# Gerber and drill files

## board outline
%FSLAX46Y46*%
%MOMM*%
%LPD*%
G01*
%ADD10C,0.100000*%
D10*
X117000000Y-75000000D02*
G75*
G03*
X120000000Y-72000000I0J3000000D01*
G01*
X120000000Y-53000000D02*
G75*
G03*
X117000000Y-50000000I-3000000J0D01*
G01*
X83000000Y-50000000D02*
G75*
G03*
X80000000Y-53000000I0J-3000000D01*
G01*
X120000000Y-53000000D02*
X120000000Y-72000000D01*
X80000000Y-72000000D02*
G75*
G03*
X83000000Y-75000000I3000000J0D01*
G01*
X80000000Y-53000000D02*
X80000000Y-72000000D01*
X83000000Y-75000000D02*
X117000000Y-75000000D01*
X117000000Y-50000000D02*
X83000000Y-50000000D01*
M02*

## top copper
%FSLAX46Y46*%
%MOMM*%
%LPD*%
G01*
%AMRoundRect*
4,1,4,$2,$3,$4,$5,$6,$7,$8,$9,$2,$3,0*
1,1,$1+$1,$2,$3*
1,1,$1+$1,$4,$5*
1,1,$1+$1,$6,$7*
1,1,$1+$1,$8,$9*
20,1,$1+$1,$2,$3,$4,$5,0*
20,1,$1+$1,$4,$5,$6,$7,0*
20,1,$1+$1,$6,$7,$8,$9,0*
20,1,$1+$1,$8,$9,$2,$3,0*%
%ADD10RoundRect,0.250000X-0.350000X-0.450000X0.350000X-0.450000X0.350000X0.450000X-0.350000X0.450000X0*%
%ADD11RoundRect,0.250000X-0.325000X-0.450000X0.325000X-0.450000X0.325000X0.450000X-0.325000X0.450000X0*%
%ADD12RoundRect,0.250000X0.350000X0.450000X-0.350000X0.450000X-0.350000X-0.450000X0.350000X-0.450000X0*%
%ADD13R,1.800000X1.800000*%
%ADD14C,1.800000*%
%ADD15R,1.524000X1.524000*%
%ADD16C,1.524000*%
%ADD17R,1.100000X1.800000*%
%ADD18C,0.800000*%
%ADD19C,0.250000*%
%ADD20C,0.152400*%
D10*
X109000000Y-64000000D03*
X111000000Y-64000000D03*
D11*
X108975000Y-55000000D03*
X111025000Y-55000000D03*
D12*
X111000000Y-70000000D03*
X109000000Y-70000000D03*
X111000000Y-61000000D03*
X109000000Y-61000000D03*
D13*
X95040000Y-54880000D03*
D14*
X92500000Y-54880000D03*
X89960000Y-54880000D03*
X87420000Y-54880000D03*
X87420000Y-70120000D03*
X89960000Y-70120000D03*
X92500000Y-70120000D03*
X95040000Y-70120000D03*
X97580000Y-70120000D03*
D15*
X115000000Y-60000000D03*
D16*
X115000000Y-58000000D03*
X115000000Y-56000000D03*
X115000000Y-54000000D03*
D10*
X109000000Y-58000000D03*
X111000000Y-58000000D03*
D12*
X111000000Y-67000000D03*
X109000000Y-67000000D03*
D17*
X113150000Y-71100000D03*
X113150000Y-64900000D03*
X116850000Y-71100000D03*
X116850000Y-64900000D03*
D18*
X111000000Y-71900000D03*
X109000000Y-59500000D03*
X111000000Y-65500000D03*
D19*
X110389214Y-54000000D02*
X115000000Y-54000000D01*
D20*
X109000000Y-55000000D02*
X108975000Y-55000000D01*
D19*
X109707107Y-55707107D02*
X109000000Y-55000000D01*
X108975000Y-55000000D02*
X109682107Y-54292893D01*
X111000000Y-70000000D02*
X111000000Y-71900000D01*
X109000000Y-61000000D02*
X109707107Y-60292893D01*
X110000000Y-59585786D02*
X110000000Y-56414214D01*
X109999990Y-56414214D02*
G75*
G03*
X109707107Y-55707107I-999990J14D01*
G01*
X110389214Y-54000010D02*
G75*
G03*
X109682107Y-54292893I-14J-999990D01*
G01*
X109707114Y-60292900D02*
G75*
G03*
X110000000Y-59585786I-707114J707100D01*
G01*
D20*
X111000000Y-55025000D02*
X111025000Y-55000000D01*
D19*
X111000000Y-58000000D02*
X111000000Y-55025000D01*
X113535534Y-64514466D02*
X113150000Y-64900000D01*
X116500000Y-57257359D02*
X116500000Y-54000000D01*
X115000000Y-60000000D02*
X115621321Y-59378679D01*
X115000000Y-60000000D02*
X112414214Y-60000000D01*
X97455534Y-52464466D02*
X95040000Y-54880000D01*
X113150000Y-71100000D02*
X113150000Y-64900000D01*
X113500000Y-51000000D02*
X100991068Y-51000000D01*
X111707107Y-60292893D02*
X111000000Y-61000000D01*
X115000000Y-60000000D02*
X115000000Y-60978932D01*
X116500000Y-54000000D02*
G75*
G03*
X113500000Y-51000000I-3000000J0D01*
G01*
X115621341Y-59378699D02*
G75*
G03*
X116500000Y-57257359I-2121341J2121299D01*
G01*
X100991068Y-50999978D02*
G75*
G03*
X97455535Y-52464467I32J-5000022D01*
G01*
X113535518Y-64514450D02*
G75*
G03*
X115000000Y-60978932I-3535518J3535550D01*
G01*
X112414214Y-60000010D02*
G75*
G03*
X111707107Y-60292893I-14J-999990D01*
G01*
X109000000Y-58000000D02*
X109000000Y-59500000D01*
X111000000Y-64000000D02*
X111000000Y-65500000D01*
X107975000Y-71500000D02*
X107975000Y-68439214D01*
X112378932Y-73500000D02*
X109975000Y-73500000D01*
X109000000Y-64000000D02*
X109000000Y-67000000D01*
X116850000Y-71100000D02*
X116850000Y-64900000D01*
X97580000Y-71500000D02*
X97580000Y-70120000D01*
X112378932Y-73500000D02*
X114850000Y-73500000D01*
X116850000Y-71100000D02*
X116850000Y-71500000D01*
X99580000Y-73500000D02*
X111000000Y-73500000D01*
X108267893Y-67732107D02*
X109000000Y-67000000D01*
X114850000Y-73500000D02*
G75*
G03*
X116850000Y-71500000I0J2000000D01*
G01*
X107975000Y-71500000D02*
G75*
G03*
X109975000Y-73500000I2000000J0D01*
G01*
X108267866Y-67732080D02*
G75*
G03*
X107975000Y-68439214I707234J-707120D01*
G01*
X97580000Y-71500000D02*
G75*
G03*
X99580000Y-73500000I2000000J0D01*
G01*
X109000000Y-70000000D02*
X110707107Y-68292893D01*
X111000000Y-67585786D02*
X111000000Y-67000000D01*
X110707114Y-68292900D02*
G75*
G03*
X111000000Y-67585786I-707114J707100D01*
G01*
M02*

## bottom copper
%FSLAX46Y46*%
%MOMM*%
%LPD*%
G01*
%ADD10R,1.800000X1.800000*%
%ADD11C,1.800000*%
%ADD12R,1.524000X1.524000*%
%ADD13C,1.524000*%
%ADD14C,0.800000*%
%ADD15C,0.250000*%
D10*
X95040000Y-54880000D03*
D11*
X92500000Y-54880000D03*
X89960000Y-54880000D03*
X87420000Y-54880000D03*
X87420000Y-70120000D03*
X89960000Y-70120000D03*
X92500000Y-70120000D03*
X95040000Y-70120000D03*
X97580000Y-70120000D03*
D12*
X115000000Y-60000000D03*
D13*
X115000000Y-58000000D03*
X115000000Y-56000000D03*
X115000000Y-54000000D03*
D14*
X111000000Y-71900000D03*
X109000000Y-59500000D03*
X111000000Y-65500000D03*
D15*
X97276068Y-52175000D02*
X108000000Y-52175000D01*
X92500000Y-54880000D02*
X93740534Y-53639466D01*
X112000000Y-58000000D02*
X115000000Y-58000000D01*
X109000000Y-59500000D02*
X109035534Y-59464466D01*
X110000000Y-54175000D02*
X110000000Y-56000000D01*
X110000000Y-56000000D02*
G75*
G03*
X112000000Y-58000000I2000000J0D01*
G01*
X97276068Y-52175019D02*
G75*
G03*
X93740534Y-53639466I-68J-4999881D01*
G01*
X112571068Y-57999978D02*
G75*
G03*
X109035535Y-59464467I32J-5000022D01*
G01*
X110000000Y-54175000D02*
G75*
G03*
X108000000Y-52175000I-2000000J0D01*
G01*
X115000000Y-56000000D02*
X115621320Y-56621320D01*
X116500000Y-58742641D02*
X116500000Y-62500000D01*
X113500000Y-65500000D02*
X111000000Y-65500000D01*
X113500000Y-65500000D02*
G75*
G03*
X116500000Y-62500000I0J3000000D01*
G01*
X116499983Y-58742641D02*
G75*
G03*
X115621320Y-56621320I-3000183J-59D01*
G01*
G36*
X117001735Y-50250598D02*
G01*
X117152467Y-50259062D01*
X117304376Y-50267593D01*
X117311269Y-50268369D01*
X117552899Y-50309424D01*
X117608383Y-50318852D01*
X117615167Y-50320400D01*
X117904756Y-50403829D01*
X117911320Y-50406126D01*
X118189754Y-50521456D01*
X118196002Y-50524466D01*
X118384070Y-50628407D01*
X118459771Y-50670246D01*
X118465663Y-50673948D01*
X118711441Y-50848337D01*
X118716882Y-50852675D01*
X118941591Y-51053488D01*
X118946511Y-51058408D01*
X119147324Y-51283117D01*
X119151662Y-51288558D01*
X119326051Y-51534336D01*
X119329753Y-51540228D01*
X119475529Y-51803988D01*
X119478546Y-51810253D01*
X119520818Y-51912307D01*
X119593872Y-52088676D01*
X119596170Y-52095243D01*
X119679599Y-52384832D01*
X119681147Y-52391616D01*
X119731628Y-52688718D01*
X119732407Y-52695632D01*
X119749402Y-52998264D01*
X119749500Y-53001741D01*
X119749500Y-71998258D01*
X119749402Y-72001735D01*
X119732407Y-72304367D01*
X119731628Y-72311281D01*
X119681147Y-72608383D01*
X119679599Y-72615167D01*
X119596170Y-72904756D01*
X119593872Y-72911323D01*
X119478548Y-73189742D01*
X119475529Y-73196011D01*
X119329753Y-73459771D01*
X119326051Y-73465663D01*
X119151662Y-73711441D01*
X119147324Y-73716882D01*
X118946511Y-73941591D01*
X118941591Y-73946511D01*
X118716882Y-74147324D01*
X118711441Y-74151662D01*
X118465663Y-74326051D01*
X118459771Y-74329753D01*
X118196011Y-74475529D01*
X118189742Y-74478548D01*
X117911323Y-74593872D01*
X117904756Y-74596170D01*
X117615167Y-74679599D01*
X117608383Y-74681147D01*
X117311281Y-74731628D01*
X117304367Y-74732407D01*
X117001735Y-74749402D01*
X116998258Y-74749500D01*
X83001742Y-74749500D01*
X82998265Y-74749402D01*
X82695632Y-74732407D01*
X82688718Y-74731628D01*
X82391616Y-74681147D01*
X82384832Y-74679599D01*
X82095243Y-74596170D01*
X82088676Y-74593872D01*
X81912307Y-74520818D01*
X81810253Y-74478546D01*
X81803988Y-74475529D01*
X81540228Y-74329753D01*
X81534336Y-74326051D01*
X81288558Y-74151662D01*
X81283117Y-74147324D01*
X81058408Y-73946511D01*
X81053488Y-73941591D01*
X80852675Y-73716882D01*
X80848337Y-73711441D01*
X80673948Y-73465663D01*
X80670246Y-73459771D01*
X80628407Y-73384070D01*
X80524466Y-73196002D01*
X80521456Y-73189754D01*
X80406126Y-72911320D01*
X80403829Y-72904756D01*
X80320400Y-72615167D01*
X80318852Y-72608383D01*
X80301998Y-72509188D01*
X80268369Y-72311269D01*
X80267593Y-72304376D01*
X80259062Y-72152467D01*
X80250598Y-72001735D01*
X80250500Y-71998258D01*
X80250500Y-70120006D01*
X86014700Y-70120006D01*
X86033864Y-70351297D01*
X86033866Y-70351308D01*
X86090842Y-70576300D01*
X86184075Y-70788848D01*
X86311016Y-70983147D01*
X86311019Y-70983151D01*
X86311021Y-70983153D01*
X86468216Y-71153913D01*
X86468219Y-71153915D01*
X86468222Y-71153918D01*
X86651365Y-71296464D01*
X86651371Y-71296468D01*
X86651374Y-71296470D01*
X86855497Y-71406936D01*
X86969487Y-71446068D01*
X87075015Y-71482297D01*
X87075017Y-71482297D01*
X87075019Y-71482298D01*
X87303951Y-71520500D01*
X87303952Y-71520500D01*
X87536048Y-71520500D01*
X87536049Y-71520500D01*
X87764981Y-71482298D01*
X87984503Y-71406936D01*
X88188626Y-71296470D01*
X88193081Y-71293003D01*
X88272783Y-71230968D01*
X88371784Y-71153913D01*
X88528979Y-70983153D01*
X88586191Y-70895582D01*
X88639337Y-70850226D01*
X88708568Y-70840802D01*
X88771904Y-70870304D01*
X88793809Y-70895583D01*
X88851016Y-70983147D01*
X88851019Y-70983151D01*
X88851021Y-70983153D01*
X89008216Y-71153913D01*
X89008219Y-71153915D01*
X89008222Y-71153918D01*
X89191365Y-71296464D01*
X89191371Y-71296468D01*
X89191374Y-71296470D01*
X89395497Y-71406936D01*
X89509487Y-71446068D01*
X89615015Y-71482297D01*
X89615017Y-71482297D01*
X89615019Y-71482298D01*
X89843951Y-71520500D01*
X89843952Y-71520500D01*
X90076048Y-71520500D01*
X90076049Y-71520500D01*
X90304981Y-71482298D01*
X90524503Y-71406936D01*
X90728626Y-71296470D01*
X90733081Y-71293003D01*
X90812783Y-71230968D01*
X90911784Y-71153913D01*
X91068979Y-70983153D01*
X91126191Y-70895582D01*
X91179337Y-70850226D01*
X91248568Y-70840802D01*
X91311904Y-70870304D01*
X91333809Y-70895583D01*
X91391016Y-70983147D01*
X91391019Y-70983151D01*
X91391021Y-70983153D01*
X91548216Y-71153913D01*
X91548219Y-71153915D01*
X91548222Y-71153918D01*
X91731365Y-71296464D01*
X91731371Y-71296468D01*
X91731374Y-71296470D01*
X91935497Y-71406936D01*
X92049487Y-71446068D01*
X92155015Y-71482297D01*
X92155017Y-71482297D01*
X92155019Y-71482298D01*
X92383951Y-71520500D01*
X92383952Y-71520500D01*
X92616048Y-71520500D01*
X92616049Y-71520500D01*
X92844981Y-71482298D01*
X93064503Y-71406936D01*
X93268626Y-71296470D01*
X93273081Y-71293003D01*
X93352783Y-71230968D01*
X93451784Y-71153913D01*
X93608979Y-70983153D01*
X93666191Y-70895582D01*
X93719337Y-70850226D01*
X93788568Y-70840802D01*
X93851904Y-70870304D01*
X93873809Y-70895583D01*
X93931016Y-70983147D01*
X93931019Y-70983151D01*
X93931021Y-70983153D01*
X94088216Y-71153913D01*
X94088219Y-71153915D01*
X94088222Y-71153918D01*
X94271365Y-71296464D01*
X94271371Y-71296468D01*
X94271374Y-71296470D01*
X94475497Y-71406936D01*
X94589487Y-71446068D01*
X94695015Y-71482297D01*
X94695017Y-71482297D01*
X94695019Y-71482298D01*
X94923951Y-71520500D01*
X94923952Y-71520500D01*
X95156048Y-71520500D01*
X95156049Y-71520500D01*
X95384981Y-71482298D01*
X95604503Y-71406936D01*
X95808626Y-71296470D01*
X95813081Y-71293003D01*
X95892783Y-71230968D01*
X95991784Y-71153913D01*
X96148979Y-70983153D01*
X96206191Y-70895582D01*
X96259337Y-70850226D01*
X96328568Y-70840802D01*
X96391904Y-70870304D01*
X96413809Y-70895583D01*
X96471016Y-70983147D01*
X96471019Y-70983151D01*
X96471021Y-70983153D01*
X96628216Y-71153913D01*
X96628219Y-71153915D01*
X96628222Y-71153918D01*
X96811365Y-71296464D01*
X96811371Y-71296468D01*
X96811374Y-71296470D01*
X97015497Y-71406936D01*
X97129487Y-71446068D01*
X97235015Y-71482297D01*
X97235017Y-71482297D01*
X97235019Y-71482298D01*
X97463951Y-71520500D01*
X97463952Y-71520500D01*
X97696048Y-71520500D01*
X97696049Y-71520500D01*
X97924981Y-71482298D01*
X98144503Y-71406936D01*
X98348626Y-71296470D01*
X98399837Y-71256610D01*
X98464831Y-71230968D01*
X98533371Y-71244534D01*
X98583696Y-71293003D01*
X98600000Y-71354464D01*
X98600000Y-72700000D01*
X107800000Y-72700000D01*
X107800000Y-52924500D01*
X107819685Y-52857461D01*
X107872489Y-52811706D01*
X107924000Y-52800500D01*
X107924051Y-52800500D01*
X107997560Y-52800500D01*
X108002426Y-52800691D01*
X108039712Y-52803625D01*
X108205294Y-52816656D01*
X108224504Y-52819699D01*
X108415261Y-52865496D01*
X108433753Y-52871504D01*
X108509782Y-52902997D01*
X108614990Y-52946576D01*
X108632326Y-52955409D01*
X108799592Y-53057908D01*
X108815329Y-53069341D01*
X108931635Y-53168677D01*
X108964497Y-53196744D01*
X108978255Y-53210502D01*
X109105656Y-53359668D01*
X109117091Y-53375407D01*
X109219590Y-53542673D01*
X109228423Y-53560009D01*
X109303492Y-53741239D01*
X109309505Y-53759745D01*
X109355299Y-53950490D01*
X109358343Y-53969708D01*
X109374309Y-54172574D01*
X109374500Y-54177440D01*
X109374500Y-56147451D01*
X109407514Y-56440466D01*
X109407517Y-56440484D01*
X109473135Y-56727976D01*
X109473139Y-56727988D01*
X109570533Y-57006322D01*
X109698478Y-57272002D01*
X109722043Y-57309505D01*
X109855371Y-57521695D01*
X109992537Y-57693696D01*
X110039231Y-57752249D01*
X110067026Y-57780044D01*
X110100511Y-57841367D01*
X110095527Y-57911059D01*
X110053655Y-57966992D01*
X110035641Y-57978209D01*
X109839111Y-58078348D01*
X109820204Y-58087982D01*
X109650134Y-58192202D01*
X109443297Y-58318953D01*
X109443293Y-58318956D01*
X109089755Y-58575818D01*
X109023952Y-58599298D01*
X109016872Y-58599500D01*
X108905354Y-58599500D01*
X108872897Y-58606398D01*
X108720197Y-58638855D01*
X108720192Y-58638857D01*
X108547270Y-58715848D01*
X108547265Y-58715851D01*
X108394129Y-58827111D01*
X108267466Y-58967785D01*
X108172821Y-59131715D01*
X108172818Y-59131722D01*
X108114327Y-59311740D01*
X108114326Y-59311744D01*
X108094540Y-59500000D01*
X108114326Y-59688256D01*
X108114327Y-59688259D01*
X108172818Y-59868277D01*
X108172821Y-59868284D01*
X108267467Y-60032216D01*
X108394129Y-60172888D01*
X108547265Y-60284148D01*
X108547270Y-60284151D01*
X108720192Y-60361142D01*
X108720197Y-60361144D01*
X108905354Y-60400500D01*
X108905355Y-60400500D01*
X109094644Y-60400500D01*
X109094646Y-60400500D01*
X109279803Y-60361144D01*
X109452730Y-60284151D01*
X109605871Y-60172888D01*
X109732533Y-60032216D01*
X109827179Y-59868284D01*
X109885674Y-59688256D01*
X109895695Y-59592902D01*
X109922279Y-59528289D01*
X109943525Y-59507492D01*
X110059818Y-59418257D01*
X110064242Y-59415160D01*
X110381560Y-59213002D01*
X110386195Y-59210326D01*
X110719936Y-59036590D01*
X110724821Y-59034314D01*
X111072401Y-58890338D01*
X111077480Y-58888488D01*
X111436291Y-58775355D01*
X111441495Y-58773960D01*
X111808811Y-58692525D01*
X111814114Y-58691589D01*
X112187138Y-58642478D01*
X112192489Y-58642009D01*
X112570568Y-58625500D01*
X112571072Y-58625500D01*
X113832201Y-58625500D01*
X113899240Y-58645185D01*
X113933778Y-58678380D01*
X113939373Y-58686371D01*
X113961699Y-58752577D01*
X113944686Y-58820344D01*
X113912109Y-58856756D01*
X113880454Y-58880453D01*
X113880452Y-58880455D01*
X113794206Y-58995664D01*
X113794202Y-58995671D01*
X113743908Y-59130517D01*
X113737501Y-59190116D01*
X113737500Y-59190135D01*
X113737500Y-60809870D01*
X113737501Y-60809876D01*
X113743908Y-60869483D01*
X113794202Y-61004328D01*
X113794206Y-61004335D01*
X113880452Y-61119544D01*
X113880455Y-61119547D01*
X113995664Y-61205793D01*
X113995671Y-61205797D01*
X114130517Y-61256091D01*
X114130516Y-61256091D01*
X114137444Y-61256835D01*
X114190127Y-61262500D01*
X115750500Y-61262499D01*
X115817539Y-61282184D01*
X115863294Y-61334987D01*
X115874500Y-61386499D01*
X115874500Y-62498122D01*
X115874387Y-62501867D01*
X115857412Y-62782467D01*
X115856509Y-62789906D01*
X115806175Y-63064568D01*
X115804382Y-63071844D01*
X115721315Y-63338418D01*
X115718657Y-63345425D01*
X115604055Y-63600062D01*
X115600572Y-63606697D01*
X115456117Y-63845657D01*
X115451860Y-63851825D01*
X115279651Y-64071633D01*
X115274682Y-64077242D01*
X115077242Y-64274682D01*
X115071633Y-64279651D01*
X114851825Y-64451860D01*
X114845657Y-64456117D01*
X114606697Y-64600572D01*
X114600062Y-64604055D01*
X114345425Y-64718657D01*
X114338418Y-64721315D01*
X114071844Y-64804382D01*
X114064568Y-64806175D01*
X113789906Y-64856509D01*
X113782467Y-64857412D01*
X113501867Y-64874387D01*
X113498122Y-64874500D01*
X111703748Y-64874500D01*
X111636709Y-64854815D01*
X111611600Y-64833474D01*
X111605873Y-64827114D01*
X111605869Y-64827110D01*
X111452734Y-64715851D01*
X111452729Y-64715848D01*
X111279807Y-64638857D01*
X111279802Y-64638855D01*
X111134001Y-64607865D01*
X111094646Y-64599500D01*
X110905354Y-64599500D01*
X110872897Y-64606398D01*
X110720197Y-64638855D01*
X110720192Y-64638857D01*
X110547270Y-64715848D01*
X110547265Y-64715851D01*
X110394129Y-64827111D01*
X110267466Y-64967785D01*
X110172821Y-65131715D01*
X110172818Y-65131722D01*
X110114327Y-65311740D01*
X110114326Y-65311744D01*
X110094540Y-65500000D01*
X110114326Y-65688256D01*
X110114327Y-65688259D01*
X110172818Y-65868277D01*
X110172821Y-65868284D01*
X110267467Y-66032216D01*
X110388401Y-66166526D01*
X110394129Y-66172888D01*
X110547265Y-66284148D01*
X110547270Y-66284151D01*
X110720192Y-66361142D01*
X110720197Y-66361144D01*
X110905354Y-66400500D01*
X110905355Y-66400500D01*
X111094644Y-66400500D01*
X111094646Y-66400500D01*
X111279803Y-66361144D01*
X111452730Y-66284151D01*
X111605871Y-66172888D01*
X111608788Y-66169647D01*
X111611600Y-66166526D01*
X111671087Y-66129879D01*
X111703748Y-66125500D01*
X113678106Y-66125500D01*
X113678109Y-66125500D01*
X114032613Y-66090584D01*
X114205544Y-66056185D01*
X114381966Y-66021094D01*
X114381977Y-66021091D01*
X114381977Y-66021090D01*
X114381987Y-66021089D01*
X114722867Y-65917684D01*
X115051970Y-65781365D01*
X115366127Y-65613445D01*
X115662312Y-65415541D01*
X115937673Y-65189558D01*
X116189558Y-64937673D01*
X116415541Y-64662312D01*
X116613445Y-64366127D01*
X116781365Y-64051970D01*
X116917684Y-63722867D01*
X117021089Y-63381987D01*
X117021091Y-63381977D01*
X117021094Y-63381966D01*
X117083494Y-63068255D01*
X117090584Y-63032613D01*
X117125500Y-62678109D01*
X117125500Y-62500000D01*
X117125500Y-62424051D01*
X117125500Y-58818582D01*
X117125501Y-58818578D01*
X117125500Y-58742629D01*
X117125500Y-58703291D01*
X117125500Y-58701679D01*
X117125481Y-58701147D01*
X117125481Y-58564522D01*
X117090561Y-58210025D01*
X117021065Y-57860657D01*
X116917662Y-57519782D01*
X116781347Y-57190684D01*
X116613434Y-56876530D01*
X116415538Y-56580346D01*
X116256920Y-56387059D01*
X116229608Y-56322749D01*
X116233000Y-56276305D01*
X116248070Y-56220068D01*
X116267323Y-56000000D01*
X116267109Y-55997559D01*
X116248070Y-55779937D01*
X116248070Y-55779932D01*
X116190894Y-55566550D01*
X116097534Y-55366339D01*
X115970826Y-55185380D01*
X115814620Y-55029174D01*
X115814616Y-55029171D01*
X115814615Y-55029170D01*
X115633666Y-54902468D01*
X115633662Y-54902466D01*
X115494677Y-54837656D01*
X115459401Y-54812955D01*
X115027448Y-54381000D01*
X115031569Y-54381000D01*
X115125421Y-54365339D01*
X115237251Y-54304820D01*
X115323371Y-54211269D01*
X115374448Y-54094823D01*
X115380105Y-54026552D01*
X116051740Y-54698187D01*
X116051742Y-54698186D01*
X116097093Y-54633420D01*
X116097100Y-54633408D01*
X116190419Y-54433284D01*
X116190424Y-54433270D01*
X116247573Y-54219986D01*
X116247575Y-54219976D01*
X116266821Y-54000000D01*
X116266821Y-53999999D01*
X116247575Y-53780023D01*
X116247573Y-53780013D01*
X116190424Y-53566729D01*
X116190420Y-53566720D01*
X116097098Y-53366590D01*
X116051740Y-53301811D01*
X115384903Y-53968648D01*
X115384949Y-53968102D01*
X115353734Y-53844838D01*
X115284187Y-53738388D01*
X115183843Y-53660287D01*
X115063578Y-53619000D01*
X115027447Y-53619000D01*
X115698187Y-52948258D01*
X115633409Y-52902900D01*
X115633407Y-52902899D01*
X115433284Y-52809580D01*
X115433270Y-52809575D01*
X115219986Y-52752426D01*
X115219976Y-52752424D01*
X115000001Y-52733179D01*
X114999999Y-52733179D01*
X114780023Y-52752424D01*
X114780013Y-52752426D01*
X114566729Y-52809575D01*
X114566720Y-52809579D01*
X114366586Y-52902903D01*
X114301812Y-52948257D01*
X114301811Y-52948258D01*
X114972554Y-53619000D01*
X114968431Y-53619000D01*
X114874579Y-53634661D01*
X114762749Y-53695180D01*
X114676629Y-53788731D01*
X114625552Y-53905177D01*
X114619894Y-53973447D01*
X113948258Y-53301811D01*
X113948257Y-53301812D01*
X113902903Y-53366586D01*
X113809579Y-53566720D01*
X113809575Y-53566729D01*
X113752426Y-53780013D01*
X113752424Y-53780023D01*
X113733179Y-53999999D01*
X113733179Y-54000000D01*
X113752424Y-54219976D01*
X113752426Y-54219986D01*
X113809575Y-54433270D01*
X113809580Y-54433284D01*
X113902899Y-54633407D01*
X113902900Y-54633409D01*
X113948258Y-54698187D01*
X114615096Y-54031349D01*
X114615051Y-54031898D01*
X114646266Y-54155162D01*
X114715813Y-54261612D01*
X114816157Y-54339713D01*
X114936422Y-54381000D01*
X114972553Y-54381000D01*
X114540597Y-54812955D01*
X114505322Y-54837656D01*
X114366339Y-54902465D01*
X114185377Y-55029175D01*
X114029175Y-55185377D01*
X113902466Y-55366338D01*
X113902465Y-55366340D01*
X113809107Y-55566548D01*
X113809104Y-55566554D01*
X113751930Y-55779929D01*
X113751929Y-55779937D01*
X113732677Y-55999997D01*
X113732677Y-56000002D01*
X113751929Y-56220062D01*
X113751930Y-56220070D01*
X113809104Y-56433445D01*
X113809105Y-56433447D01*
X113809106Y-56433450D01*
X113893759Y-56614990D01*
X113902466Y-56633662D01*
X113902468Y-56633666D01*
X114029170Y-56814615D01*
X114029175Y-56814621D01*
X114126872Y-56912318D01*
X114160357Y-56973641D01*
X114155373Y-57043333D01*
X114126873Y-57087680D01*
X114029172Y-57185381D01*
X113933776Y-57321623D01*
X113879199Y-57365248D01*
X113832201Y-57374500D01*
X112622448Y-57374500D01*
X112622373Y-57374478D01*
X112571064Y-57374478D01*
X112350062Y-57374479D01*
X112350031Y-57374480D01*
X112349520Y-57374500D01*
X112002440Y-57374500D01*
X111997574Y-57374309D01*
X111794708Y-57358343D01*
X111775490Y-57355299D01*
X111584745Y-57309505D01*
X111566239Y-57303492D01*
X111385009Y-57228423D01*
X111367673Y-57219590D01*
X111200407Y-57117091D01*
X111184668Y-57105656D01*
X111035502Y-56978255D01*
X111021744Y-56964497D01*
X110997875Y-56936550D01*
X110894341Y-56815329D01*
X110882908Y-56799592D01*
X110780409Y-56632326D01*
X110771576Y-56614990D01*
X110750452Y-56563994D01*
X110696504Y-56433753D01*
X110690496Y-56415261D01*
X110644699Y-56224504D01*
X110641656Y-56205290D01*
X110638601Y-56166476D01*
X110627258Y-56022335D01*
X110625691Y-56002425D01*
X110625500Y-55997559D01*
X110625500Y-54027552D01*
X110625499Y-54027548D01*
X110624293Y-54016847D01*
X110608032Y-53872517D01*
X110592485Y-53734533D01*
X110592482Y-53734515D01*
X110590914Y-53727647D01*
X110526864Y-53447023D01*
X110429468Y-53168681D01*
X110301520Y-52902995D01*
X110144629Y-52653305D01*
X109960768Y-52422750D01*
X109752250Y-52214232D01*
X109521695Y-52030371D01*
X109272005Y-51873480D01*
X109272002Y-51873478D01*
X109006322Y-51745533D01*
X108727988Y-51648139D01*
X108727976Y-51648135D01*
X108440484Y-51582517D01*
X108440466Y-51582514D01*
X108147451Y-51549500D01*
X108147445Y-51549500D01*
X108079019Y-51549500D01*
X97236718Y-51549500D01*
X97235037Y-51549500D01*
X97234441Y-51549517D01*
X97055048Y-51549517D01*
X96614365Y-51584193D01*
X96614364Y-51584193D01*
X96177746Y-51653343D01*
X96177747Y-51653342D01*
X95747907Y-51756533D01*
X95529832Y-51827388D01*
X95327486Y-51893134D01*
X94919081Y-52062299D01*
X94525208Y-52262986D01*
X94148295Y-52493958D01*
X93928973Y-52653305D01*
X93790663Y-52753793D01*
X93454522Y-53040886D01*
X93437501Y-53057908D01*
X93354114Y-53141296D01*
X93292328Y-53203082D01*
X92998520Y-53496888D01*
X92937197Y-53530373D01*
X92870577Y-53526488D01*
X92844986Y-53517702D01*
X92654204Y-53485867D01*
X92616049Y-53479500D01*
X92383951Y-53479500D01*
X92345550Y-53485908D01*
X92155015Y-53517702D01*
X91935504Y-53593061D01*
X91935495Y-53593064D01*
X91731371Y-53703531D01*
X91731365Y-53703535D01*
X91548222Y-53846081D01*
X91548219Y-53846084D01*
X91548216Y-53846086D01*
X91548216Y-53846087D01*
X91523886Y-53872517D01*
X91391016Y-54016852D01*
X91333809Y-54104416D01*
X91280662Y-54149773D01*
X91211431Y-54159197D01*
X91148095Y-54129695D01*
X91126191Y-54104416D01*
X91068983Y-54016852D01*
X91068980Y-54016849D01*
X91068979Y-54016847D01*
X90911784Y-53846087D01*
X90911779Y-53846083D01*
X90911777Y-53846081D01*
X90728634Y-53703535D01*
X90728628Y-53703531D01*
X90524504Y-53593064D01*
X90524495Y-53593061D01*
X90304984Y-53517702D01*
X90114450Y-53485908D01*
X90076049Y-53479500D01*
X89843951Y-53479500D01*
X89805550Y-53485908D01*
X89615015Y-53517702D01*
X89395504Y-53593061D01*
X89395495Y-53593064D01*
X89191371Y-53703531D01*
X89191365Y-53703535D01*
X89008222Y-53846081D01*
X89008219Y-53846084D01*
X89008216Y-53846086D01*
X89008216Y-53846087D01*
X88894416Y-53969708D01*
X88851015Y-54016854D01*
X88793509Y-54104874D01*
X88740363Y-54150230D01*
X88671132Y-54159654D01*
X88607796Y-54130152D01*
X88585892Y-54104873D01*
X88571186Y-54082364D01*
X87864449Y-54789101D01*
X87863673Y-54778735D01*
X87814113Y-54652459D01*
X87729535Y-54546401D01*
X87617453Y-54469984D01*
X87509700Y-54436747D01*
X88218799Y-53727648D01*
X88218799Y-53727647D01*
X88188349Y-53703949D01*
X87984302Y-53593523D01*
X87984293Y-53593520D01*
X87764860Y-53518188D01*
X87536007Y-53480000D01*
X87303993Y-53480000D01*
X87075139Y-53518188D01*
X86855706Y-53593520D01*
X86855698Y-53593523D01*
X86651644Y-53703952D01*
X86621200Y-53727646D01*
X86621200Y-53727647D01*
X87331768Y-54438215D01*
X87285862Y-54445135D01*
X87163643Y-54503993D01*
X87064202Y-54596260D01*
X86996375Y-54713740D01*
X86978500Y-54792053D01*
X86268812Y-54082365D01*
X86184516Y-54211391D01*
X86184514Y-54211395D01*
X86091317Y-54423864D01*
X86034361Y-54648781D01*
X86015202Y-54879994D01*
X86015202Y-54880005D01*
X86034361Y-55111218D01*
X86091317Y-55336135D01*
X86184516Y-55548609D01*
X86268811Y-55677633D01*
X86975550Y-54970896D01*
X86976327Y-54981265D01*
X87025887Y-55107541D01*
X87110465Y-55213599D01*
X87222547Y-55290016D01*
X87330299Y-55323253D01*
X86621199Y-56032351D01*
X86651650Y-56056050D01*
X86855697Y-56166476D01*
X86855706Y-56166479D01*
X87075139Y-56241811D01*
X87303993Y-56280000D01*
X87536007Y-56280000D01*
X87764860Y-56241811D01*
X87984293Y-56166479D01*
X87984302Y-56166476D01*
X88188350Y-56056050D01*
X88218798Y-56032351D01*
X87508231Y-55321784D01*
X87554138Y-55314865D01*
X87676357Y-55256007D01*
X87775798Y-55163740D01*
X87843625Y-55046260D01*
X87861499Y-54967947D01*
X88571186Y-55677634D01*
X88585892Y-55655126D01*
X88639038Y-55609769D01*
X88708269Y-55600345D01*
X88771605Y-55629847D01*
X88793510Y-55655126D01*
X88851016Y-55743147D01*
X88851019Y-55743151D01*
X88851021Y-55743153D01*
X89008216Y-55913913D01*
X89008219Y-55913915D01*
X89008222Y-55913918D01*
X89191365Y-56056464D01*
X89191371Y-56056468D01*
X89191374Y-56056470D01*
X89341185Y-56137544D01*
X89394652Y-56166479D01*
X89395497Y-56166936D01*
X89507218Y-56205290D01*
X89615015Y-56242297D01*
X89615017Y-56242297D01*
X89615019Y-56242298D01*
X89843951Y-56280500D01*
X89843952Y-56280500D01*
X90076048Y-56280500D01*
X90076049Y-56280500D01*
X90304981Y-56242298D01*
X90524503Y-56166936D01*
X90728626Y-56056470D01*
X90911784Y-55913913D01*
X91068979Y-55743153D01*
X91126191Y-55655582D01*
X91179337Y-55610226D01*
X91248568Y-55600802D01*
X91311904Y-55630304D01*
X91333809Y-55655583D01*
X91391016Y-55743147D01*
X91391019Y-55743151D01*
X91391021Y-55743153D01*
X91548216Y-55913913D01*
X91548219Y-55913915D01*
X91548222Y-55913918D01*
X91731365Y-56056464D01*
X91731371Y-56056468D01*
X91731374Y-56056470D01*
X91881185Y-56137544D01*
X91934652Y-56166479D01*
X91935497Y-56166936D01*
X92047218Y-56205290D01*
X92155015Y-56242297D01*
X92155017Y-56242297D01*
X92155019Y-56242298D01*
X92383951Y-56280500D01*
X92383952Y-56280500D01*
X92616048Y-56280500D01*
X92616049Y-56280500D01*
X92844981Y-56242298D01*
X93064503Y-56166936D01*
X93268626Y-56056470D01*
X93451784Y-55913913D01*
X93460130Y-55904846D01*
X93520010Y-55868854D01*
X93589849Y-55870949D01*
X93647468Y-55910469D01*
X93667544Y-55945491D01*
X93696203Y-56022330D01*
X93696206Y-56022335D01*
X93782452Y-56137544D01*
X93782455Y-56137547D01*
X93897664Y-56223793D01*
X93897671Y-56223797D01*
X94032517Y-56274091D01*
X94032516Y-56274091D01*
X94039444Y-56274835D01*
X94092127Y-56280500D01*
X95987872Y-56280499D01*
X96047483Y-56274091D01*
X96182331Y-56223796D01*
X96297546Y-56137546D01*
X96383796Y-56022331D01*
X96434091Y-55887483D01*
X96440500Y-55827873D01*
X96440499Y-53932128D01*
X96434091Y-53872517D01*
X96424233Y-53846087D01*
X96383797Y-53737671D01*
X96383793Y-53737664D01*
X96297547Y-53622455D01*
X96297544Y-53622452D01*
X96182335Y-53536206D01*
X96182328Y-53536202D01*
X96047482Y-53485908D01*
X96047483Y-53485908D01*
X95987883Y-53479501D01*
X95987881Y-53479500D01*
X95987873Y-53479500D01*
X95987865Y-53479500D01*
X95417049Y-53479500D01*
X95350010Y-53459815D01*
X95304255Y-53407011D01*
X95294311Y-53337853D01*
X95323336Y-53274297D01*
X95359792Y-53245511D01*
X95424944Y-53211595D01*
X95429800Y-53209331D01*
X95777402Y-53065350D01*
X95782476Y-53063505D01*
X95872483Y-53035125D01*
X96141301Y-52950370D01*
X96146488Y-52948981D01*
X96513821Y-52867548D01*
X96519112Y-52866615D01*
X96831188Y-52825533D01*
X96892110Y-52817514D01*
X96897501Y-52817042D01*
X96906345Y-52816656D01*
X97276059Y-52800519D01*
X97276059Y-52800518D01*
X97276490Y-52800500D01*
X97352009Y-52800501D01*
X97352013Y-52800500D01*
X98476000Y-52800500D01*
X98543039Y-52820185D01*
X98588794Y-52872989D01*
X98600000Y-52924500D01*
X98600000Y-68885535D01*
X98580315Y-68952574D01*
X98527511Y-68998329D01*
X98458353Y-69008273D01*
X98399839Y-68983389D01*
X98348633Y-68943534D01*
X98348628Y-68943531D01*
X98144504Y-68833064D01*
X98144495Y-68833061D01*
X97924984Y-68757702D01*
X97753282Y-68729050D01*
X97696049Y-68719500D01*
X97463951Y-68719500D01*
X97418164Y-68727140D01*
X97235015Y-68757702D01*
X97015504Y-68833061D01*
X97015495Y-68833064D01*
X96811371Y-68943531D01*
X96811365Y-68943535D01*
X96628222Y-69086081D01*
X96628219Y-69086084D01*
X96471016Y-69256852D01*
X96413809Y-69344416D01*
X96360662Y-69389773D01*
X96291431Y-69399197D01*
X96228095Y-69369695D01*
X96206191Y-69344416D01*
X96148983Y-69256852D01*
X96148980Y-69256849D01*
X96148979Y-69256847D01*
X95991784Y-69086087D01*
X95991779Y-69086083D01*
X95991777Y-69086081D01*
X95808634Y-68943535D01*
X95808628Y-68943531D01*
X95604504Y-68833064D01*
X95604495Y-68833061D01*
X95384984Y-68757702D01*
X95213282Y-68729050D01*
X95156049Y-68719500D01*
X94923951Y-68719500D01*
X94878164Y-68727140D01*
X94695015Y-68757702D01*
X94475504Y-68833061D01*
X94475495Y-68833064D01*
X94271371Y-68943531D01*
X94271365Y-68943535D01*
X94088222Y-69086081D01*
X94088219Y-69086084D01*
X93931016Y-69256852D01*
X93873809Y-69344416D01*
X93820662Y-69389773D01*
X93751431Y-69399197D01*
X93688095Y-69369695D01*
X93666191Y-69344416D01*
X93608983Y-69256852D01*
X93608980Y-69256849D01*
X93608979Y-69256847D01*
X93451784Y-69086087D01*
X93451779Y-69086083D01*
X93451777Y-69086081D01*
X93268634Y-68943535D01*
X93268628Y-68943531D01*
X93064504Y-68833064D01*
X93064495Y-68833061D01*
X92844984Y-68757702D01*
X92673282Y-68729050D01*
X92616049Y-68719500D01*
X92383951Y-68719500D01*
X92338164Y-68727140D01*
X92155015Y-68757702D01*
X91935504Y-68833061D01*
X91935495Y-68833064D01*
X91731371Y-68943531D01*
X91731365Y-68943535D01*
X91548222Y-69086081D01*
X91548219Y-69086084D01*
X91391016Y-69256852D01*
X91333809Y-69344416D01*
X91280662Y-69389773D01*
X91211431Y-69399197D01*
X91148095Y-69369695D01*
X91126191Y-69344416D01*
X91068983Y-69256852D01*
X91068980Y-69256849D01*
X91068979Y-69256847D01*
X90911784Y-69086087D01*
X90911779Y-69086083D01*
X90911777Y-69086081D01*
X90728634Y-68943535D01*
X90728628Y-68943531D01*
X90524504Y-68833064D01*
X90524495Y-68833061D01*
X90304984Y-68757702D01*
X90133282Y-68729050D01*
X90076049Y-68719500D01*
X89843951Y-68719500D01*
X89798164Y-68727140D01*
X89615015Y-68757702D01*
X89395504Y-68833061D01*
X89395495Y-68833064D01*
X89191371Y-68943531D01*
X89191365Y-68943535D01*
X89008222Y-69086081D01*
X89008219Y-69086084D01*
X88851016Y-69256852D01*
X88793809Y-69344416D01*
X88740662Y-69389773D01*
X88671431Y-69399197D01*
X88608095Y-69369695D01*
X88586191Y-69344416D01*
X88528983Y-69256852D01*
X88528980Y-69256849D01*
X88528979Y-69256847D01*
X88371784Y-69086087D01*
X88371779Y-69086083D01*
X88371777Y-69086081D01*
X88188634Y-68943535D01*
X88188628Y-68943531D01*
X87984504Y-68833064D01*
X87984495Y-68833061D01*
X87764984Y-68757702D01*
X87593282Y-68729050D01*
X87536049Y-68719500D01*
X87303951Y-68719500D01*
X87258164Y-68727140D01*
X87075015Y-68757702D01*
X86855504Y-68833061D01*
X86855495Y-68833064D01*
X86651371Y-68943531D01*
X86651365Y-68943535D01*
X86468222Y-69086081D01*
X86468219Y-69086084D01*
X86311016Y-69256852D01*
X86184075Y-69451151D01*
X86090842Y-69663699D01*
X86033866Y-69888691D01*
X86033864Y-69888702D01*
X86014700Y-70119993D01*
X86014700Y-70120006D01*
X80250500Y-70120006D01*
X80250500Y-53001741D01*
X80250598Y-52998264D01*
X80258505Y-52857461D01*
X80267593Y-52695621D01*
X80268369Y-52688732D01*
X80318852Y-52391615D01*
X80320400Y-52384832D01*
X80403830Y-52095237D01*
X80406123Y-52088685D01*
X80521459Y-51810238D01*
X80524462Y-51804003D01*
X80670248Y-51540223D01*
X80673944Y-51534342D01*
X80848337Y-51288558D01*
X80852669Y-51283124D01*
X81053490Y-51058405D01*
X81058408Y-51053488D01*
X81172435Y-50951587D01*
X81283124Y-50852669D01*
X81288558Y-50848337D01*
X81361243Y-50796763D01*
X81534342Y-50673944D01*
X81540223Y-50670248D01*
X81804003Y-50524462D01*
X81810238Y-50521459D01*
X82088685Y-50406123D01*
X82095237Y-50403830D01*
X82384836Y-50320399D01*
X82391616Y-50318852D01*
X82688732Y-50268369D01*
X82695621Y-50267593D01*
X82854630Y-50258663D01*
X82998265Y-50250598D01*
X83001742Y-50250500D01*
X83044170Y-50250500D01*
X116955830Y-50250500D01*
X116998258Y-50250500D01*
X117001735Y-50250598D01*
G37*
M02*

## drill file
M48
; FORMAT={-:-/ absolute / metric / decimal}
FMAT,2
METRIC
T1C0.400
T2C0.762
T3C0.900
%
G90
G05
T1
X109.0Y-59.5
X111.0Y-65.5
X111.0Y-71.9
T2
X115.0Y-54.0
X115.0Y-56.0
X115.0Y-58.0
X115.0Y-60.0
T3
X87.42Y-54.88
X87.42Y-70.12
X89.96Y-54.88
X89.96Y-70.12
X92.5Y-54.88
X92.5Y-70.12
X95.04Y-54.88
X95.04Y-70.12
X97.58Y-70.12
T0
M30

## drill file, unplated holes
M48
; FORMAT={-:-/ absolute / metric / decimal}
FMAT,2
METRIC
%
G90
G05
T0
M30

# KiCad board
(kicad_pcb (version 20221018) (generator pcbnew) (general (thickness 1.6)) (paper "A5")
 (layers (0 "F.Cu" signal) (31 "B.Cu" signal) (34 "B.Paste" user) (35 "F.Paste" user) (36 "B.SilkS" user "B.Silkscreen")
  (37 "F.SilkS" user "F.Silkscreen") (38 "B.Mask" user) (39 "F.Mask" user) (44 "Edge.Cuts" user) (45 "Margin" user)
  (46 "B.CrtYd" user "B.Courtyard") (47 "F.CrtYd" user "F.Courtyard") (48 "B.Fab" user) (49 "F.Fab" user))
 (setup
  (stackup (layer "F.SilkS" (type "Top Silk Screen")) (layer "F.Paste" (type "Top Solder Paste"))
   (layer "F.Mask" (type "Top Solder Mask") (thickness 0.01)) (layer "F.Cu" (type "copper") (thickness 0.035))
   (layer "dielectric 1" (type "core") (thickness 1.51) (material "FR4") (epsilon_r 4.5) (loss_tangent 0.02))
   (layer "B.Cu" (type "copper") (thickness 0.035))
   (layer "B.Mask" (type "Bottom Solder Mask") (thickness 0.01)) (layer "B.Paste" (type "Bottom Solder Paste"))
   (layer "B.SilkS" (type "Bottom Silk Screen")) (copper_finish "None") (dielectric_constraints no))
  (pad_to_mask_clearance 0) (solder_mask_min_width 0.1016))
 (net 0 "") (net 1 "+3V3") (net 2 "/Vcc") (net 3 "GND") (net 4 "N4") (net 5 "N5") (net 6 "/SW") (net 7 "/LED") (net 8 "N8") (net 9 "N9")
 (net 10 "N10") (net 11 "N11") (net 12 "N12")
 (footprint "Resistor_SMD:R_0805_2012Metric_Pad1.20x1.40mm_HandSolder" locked (layer "F.Cu") (at 110 64)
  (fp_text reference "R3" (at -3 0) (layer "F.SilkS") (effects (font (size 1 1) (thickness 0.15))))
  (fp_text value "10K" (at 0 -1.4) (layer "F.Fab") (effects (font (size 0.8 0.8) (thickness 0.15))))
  (pad "1" smd roundrect locked (at -1 0) (size 1.2 1.4) (layers "F.Cu" "F.Paste" "F.Mask") (roundrect_rratio 0.2083333333) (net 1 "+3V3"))
  (pad "2" smd roundrect locked (at 1 0) (size 1.2 1.4) (layers "F.Cu" "F.Paste" "F.Mask") (roundrect_rratio 0.2083333333) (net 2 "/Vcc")))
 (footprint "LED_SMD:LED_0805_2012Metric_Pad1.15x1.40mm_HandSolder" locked (layer "F.Cu") (at 110 55)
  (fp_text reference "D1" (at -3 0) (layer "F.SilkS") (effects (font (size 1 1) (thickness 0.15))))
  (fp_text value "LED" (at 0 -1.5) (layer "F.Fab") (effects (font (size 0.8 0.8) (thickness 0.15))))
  (pad "1" smd roundrect locked (at -1.025 0) (size 1.15 1.4) (layers "F.Cu" "F.Paste" "F.Mask") (roundrect_rratio 0.2173913043)
   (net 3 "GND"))
  (pad "2" smd roundrect locked (at 1.025 0) (size 1.15 1.4) (layers "F.Cu" "F.Paste" "F.Mask") (roundrect_rratio 0.2173913043) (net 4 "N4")))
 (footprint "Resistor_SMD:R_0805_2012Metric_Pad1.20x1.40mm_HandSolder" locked (layer "F.Cu") (at 110 70 180)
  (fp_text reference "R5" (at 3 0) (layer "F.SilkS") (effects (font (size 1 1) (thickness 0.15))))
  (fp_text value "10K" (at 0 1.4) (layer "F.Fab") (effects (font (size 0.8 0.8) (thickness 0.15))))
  (pad "1" smd roundrect locked (at -1 0 180) (size 1.2 1.4) (layers "F.Cu" "F.Paste" "F.Mask") (roundrect_rratio 0.2083333333)
   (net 3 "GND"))
  (pad "2" smd roundrect locked (at 1 0 180) (size 1.2 1.4) (layers "F.Cu" "F.Paste" "F.Mask") (roundrect_rratio 0.2083333333) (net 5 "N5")))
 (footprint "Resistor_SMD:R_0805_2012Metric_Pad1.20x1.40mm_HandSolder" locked (layer "F.Cu") (at 110 61 180)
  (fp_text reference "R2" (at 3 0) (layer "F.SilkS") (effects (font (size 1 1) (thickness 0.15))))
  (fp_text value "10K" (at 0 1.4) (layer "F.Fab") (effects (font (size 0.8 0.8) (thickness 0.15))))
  (pad "1" smd roundrect locked (at -1 0 180) (size 1.2 1.4) (layers "F.Cu" "F.Paste" "F.Mask") (roundrect_rratio 0.2083333333)
   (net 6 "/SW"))
  (pad "2" smd roundrect locked (at 1 0 180) (size 1.2 1.4) (layers "F.Cu" "F.Paste" "F.Mask") (roundrect_rratio 0.2083333333) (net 3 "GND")))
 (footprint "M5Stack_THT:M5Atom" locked (layer "F.Cu") (at 92.5 62.5 -90)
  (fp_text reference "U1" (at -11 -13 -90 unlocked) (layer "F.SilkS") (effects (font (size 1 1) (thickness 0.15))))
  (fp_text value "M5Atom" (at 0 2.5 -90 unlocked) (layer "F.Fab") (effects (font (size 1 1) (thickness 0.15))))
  (pad "1" thru_hole rect locked (at -7.62 -2.54 270) (size 1.8 1.8) (drill 0.9) (layers "*.Cu" "*.Mask") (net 6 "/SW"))
  (pad "2" thru_hole circle locked (at -7.62 0 270) (size 1.8 1.8) (drill 0.9) (layers "*.Cu" "*.Mask") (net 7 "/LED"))
  (pad "3" thru_hole circle locked (at -7.62 2.54 270) (size 1.8 1.8) (drill 0.9) (layers "*.Cu" "*.Mask") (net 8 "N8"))
  (pad "4" thru_hole circle locked (at -7.62 5.08 270) (size 1.8 1.8) (drill 0.9) (layers "*.Cu" "*.Mask") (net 3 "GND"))
  (pad "5" thru_hole circle locked (at 7.62 5.08 270) (size 1.8 1.8) (drill 0.9) (layers "*.Cu" "*.Mask") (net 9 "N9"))
  (pad "6" thru_hole circle locked (at 7.62 2.54 270) (size 1.8 1.8) (drill 0.9) (layers "*.Cu" "*.Mask") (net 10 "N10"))
  (pad "7" thru_hole circle locked (at 7.62 0 270) (size 1.8 1.8) (drill 0.9) (layers "*.Cu" "*.Mask") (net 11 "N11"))
  (pad "8" thru_hole circle locked (at 7.62 -2.54 270) (size 1.8 1.8) (drill 0.9) (layers "*.Cu" "*.Mask") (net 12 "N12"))
  (pad "9" thru_hole circle locked (at 7.62 -5.08 270) (size 1.8 1.8) (drill 0.9) (layers "*.Cu" "*.Mask") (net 1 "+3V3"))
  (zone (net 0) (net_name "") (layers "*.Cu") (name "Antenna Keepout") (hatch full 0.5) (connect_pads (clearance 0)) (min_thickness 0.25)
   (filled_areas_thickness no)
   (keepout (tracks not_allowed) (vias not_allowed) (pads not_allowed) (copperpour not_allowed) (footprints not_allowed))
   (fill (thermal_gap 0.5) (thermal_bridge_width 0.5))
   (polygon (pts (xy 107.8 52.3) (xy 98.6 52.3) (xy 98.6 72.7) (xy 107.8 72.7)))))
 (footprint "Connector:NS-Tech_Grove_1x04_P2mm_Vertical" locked (layer "F.Cu") (at 115 60 180)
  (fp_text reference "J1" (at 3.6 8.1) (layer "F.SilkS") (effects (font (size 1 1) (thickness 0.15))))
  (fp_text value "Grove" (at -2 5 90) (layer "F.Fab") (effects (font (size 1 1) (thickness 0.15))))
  (pad "1" thru_hole rect locked (at 0 0 180) (size 1.524 1.524) (drill 0.762) (layers "*.Cu" "*.Mask") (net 6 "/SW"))
  (pad "2" thru_hole circle locked (at 0 2 180) (size 1.524 1.524) (drill 0.762) (layers "*.Cu" "*.Mask") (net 7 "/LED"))
  (pad "3" thru_hole circle locked (at 0 4 180) (size 1.524 1.524) (drill 0.762) (layers "*.Cu" "*.Mask") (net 2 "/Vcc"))
  (pad "4" thru_hole circle locked (at 0 6 180) (size 1.524 1.524) (drill 0.762) (layers "*.Cu" "*.Mask") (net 3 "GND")))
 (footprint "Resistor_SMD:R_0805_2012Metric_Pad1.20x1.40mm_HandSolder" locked (layer "F.Cu") (at 110 58)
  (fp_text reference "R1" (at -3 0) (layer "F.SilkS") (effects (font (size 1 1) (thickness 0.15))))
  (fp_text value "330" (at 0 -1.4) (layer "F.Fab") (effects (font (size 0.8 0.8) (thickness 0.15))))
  (pad "1" smd roundrect locked (at -1 0) (size 1.2 1.4) (layers "F.Cu" "F.Paste" "F.Mask") (roundrect_rratio 0.2083333333) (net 7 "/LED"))
  (pad "2" smd roundrect locked (at 1 0) (size 1.2 1.4) (layers "F.Cu" "F.Paste" "F.Mask") (roundrect_rratio 0.2083333333) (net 4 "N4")))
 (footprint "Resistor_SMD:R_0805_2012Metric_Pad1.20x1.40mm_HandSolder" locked (layer "F.Cu") (at 110 67 180)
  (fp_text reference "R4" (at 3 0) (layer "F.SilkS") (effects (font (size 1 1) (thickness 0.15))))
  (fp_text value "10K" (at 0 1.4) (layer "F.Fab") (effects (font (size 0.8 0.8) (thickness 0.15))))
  (pad "1" smd roundrect locked (at -1 0 180) (size 1.2 1.4) (layers "F.Cu" "F.Paste" "F.Mask") (roundrect_rratio 0.2083333333) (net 5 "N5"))
  (pad "2" smd roundrect locked (at 1 0 180) (size 1.2 1.4) (layers "F.Cu" "F.Paste" "F.Mask") (roundrect_rratio 0.2083333333)
   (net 1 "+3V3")))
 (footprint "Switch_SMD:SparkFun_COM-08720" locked (layer "F.Cu") (at 115 68 90)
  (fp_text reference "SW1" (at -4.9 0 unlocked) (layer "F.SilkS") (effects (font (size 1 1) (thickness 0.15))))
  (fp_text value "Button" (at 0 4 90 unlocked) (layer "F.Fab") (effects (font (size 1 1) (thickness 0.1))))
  (pad "1" smd rect locked (at -3.1 -1.85 90) (size 1.8 1.1) (layers "F.Cu" "F.Paste" "F.Mask") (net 6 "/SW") (thermal_bridge_angle 45))
  (pad "1" smd rect locked (at 3.1 -1.85 90) (size 1.8 1.1) (layers "F.Cu" "F.Paste" "F.Mask") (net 6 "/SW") (thermal_bridge_angle 45))
  (pad "2" smd rect locked (at -3.1 1.85 90) (size 1.8 1.1) (layers "F.Cu" "F.Paste" "F.Mask") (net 1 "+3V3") (thermal_bridge_angle 45))
  (pad "2" smd rect locked (at 3.1 1.85 90) (size 1.8 1.1) (layers "F.Cu" "F.Paste" "F.Mask") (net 1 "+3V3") (thermal_bridge_angle 45)))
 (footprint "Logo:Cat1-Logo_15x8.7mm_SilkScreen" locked (layer "B.Cu") (at 108.8 70.5 180)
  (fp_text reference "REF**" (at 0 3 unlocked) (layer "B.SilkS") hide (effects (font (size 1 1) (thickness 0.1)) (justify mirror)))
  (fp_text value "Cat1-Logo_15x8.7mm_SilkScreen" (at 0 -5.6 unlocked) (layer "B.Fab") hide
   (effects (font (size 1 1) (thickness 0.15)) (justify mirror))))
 (gr_arc locked (start 120 72) (mid 119.12132 74.12132) (end 117 75) (stroke (width 0.1) (type default)) (layer "Edge.Cuts"))
 (gr_arc locked (start 117 50) (mid 119.12132 50.87868) (end 120 53) (stroke (width 0.1) (type default)) (layer "Edge.Cuts"))
 (gr_arc locked (start 80 53) (mid 80.87868 50.87868) (end 83 50) (stroke (width 0.1) (type default)) (layer "Edge.Cuts"))
 (gr_line locked (start 120 53) (end 120 72) (stroke (width 0.1) (type default)) (layer "Edge.Cuts"))
 (gr_arc locked (start 83 75) (mid 80.87868 74.12132) (end 80 72) (stroke (width 0.1) (type default)) (layer "Edge.Cuts"))
 (gr_line locked (start 80 53) (end 80 72) (stroke (width 0.1) (type default)) (layer "Edge.Cuts"))
 (gr_line locked (start 83 75) (end 117 75) (stroke (width 0.1) (type default)) (layer "Edge.Cuts"))
 (gr_line locked (start 117 50) (end 83 50) (stroke (width 0.1) (type default)) (layer "Edge.Cuts"))
 (segment (start 110.389214 54) (end 115 54) (width 0.25) (layer "F.Cu") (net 3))
 (segment (start 109 55) (end 108.975 55) (width 0.1524) (layer "F.Cu") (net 3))
 (segment (start 109.707107 55.707107) (end 109 55) (width 0.25) (layer "F.Cu") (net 3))
 (segment (start 108.975 55) (end 109.682107 54.292893) (width 0.25) (layer "F.Cu") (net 3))
 (segment (start 111 70) (end 111 71.9) (width 0.25) (layer "F.Cu") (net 3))
 (segment (start 109 61) (end 109.707107 60.292893) (width 0.25) (layer "F.Cu") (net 3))
 (segment (start 110 59.585786) (end 110 56.414214) (width 0.25) (layer "F.Cu") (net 3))
 (via (at 111 71.9) (size 0.8) (drill 0.4) (layers "F.Cu" "B.Cu") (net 3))
 (arc (start 109.707107 55.707107) (mid 109.92388 56.03153) (end 110 56.414214) (width 0.25) (layer "F.Cu") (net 3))
 (arc (start 110.389214 54) (mid 110.006531 54.07612) (end 109.682107 54.292893) (width 0.25) (layer "F.Cu") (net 3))
 (arc (start 109.707107 60.292893) (mid 109.92388 59.96847) (end 110 59.585786) (width 0.25) (layer "F.Cu") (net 3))
 (segment (start 111 55.025) (end 111.025 55) (width 0.1524) (layer "F.Cu") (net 4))
 (segment (start 111 58) (end 111 55.025) (width 0.25) (layer "F.Cu") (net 4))
 (segment (start 113.535534 64.514466) (end 113.15 64.9) (width 0.25) (layer "F.Cu") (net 6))
 (segment (start 116.5 57.257359) (end 116.5 54) (width 0.25) (layer "F.Cu") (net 6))
 (segment (start 115 60) (end 115.621321 59.378679) (width 0.25) (layer "F.Cu") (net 6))
 (segment (start 115 60) (end 112.414214 60) (width 0.25) (layer "F.Cu") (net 6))
 (segment (start 97.455534 52.464466) (end 95.04 54.88) (width 0.25) (layer "F.Cu") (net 6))
 (segment (start 113.15 71.1) (end 113.15 64.9) (width 0.25) (layer "F.Cu") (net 6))
 (segment (start 113.5 51) (end 100.991068 51) (width 0.25) (layer "F.Cu") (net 6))
 (segment (start 111.707107 60.292893) (end 111 61) (width 0.25) (layer "F.Cu") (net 6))
 (segment (start 115 60) (end 115 60.978932) (width 0.25) (layer "F.Cu") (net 6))
 (arc (start 116.5 54) (mid 115.62132 51.87868) (end 113.5 51) (width 0.25) (layer "F.Cu") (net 6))
 (arc (start 116.5 57.257359) (mid 116.271639 58.405409) (end 115.621321 59.378679) (width 0.25) (layer "F.Cu") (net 6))
 (arc (start 97.455534 52.464466) (mid 99.077651 51.380602) (end 100.991068 51) (width 0.25) (layer "F.Cu") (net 6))
 (arc (start 113.535534 64.514466) (mid 114.619398 62.892349) (end 115 60.978932) (width 0.25) (layer "F.Cu") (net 6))
 (arc (start 112.414214 60) (mid 112.031531 60.07612) (end 111.707107 60.292893) (width 0.25) (layer "F.Cu") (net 6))
 (segment (start 109 58) (end 109 59.5) (width 0.25) (layer "F.Cu") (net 7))
 (via (at 109 59.5) (size 0.8) (drill 0.4) (layers "F.Cu" "B.Cu") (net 7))
 (segment (start 97.276068 52.175) (end 108 52.175) (width 0.25) (layer "B.Cu") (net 7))
 (segment (start 92.5 54.88) (end 93.740534 53.639466) (width 0.25) (layer "B.Cu") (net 7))
 (segment (start 112 58) (end 115 58) (width 0.25) (layer "B.Cu") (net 7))
 (segment (start 109 59.5) (end 109.035534 59.464466) (width 0.25) (layer "B.Cu") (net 7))
 (segment (start 110 54.175) (end 110 56) (width 0.25) (layer "B.Cu") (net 7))
 (arc (start 110 56) (mid 110.585786 57.414214) (end 112 58) (width 0.25) (layer "B.Cu") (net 7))
 (arc (start 93.740534 53.639466) (mid 95.362649 52.555592) (end 97.276068 52.175) (width 0.25) (layer "B.Cu") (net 7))
 (arc (start 112.571068 58) (mid 110.657651 58.380602) (end 109.035534 59.464466) (width 0.25) (layer "B.Cu") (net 7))
 (arc (start 108 52.175) (mid 109.414214 52.760786) (end 110 54.175) (width 0.25) (layer "B.Cu") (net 7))
 (segment (start 111 64) (end 111 65.5) (width 0.25) (layer "F.Cu") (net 2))
 (via (at 111 65.5) (size 0.8) (drill 0.4) (layers "F.Cu" "B.Cu") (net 2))
 (segment (start 115 56) (end 115.62132 56.62132) (width 0.25) (layer "B.Cu") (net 2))
 (segment (start 116.5 58.742641) (end 116.5 62.5) (width 0.25) (layer "B.Cu") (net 2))
 (segment (start 113.5 65.5) (end 111 65.5) (width 0.25) (layer "B.Cu") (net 2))
 (arc (start 116.5 62.5) (mid 115.62132 64.62132) (end 113.5 65.5) (width 0.25) (layer "B.Cu") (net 2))
 (arc (start 115.62132 56.62132) (mid 116.271625 57.594593) (end 116.5 58.742641) (width 0.25) (layer "B.Cu") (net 2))
 (segment (start 107.975 71.5) (end 107.975 68.439214) (width 0.25) (layer "F.Cu") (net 1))
 (segment (start 112.378932 73.5) (end 109.975 73.5) (width 0.25) (layer "F.Cu") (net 1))
 (segment (start 109 64) (end 109 67) (width 0.25) (layer "F.Cu") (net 1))
 (segment (start 116.85 71.1) (end 116.85 64.9) (width 0.25) (layer "F.Cu") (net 1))
 (segment (start 97.58 71.5) (end 97.58 70.12) (width 0.25) (layer "F.Cu") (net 1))
 (segment (start 112.378932 73.5) (end 114.85 73.5) (width 0.25) (layer "F.Cu") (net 1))
 (segment (start 116.85 71.1) (end 116.85 71.5) (width 0.25) (layer "F.Cu") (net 1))
 (segment (start 99.58 73.5) (end 111 73.5) (width 0.25) (layer "F.Cu") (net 1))
 (segment (start 108.267893 67.732107) (end 109 67) (width 0.25) (layer "F.Cu") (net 1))
 (arc (start 116.85 71.5) (mid 116.264214 72.914214) (end 114.85 73.5) (width 0.25) (layer "F.Cu") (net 1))
 (arc (start 109.975 73.5) (mid 108.560786 72.914214) (end 107.975 71.5) (width 0.25) (layer "F.Cu") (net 1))
 (arc (start 107.975 68.439214) (mid 108.051125 68.056531) (end 108.267893 67.732107) (width 0.25) (layer "F.Cu") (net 1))
 (arc (start 97.58 71.5) (mid 98.165786 72.914214) (end 99.58 73.5) (width 0.25) (layer "F.Cu") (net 1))
 (segment (start 109 70) (end 110.707107 68.292893) (width 0.25) (layer "F.Cu") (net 5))
 (segment (start 111 67.585786) (end 111 67) (width 0.25) (layer "F.Cu") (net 5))
 (arc (start 111 67.585786) (mid 110.92388 67.968469) (end 110.707107 68.292893) (width 0.25) (layer "F.Cu") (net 5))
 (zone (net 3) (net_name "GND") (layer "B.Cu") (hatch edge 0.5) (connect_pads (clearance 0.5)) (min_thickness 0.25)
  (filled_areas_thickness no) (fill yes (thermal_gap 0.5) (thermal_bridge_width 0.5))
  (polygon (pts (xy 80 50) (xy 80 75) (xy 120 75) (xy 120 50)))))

